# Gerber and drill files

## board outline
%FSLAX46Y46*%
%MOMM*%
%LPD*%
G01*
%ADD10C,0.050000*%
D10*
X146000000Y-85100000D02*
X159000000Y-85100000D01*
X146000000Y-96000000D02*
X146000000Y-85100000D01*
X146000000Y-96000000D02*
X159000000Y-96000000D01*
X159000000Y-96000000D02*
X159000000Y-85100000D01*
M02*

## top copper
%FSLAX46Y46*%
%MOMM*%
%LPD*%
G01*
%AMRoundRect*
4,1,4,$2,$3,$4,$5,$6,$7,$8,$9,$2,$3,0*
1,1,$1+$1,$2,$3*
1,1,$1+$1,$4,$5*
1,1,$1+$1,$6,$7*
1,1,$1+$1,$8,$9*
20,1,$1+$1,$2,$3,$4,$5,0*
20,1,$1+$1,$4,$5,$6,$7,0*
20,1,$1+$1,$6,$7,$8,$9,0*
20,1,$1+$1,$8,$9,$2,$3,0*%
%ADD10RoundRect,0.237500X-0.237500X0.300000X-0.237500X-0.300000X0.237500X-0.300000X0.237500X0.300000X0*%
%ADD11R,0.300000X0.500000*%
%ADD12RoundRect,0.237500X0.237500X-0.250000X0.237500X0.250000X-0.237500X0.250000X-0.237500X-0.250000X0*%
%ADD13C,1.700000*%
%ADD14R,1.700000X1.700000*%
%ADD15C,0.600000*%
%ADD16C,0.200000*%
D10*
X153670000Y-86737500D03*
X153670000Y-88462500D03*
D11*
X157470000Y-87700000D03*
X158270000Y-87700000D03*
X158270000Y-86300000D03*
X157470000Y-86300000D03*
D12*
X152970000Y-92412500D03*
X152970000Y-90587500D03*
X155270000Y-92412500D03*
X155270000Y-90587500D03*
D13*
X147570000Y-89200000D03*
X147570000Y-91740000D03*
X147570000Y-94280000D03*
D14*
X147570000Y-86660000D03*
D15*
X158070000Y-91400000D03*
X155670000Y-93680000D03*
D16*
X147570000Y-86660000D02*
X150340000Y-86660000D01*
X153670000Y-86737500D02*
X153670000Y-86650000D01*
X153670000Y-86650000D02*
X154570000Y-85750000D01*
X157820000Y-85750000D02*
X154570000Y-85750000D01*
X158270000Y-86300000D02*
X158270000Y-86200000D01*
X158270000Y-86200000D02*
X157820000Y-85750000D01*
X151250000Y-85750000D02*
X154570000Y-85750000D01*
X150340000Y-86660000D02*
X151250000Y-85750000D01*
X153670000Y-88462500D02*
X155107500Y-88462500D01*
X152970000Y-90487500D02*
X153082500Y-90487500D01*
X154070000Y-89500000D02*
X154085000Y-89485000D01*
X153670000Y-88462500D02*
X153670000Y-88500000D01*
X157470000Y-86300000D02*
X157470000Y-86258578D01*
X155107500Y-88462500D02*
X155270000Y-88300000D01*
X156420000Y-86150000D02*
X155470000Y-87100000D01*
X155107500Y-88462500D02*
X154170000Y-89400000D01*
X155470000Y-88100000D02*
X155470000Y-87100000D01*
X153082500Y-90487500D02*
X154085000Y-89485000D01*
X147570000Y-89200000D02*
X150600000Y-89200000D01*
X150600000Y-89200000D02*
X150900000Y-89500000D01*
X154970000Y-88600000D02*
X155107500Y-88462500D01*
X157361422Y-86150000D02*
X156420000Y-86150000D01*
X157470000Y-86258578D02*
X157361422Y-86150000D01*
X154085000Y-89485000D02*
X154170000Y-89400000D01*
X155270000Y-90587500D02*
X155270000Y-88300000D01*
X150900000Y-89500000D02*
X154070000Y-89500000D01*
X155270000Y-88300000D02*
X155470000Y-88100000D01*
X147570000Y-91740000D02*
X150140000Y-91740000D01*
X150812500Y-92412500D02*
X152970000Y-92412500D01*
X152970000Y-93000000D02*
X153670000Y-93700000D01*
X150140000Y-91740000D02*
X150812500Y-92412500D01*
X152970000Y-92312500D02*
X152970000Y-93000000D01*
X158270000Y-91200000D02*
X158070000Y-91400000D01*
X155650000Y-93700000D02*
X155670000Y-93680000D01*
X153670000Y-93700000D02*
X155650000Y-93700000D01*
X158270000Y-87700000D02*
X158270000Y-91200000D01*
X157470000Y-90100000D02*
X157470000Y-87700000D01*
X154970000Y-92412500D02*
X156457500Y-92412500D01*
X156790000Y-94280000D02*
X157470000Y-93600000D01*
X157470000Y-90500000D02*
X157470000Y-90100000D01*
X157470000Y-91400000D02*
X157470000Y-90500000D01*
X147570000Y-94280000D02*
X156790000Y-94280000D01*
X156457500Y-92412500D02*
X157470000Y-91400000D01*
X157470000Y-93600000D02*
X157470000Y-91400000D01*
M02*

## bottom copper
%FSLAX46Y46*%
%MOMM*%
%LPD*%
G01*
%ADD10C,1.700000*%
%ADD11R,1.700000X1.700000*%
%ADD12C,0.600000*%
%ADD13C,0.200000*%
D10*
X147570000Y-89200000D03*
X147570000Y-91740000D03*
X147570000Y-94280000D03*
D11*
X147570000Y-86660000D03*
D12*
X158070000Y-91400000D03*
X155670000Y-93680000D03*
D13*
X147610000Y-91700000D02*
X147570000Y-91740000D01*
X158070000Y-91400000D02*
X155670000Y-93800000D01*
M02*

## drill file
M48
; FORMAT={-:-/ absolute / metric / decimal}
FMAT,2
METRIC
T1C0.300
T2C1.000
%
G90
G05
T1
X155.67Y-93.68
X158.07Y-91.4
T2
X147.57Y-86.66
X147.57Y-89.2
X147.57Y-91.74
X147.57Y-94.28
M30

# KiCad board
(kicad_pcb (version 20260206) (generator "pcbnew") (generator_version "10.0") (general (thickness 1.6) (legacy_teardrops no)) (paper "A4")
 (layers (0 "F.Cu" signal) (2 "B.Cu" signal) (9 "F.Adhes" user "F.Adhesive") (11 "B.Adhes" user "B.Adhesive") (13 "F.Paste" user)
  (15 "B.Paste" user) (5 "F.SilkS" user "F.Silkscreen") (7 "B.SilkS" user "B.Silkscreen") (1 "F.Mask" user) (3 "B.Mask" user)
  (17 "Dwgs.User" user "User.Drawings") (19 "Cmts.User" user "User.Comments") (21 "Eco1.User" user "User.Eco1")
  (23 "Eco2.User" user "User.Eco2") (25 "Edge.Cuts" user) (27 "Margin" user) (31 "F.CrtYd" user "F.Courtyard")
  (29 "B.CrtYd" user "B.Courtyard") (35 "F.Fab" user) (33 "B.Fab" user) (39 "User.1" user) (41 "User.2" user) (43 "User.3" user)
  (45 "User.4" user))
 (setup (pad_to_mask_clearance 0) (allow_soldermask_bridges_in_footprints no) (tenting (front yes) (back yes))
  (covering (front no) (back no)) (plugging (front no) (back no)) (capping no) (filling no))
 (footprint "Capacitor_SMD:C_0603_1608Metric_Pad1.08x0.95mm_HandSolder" (layer "F.Cu") (at 153.67 87.6 -90)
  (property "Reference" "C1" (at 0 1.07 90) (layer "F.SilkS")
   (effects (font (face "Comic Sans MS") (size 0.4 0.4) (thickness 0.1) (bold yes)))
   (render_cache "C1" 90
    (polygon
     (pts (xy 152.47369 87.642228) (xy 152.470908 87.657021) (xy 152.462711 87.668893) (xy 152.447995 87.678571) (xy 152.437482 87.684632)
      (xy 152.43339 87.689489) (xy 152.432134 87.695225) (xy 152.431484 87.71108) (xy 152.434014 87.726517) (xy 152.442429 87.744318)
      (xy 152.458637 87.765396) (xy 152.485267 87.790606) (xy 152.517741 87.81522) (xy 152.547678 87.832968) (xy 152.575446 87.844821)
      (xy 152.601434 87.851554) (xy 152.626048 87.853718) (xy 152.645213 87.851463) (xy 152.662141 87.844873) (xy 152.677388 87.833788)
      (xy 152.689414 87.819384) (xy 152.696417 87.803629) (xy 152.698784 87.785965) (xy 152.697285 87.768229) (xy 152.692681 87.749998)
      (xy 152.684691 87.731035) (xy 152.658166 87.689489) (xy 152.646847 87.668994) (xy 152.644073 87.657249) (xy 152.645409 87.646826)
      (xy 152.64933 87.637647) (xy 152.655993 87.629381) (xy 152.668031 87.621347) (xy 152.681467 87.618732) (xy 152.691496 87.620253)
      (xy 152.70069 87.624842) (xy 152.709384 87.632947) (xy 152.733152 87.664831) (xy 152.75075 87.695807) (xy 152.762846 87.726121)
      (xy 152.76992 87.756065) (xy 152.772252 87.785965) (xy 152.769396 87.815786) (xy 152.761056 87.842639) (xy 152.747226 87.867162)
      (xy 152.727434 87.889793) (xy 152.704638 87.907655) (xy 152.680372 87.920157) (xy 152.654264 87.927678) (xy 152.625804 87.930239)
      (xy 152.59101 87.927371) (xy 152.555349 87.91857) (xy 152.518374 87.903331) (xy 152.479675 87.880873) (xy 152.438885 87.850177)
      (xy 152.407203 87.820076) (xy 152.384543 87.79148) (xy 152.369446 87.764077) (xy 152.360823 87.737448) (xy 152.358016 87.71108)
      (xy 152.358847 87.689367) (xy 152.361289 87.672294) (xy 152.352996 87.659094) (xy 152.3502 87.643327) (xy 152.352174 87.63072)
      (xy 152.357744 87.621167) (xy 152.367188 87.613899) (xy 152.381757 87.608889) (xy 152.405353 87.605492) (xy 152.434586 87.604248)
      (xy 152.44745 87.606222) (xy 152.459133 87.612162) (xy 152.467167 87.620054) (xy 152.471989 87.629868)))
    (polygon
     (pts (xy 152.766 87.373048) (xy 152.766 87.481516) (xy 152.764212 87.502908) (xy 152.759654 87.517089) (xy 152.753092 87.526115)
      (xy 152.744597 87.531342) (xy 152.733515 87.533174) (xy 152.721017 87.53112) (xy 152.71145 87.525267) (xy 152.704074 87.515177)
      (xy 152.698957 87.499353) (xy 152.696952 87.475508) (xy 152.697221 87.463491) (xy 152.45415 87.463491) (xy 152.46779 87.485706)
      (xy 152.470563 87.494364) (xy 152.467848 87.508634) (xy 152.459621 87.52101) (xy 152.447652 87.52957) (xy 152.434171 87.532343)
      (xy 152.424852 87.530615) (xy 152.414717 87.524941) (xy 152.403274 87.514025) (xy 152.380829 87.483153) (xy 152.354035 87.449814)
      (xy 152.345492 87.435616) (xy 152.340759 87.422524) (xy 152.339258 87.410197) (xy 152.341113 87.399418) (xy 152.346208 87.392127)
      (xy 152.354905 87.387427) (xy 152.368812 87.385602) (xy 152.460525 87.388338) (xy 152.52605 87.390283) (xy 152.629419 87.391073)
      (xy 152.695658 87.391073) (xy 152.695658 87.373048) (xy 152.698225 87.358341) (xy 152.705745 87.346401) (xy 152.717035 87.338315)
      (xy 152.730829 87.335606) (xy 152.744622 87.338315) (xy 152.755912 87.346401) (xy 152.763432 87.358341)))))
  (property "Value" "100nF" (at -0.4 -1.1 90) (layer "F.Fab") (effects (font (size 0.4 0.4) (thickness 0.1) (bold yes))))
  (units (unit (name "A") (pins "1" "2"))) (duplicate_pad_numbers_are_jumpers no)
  (pad "1" smd roundrect (at -0.8625 0 270) (size 1.075 0.95) (layers "F.Cu" "F.Mask" "F.Paste") (roundrect_rratio 0.25)
   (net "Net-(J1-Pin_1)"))
  (pad "2" smd roundrect (at 0.8625 0 270) (size 1.075 0.95) (layers "F.Cu" "F.Mask" "F.Paste") (roundrect_rratio 0.25)
   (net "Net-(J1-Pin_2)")))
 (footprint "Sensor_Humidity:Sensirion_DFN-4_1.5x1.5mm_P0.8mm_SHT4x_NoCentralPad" (layer "F.Cu") (at 157.87 87 90)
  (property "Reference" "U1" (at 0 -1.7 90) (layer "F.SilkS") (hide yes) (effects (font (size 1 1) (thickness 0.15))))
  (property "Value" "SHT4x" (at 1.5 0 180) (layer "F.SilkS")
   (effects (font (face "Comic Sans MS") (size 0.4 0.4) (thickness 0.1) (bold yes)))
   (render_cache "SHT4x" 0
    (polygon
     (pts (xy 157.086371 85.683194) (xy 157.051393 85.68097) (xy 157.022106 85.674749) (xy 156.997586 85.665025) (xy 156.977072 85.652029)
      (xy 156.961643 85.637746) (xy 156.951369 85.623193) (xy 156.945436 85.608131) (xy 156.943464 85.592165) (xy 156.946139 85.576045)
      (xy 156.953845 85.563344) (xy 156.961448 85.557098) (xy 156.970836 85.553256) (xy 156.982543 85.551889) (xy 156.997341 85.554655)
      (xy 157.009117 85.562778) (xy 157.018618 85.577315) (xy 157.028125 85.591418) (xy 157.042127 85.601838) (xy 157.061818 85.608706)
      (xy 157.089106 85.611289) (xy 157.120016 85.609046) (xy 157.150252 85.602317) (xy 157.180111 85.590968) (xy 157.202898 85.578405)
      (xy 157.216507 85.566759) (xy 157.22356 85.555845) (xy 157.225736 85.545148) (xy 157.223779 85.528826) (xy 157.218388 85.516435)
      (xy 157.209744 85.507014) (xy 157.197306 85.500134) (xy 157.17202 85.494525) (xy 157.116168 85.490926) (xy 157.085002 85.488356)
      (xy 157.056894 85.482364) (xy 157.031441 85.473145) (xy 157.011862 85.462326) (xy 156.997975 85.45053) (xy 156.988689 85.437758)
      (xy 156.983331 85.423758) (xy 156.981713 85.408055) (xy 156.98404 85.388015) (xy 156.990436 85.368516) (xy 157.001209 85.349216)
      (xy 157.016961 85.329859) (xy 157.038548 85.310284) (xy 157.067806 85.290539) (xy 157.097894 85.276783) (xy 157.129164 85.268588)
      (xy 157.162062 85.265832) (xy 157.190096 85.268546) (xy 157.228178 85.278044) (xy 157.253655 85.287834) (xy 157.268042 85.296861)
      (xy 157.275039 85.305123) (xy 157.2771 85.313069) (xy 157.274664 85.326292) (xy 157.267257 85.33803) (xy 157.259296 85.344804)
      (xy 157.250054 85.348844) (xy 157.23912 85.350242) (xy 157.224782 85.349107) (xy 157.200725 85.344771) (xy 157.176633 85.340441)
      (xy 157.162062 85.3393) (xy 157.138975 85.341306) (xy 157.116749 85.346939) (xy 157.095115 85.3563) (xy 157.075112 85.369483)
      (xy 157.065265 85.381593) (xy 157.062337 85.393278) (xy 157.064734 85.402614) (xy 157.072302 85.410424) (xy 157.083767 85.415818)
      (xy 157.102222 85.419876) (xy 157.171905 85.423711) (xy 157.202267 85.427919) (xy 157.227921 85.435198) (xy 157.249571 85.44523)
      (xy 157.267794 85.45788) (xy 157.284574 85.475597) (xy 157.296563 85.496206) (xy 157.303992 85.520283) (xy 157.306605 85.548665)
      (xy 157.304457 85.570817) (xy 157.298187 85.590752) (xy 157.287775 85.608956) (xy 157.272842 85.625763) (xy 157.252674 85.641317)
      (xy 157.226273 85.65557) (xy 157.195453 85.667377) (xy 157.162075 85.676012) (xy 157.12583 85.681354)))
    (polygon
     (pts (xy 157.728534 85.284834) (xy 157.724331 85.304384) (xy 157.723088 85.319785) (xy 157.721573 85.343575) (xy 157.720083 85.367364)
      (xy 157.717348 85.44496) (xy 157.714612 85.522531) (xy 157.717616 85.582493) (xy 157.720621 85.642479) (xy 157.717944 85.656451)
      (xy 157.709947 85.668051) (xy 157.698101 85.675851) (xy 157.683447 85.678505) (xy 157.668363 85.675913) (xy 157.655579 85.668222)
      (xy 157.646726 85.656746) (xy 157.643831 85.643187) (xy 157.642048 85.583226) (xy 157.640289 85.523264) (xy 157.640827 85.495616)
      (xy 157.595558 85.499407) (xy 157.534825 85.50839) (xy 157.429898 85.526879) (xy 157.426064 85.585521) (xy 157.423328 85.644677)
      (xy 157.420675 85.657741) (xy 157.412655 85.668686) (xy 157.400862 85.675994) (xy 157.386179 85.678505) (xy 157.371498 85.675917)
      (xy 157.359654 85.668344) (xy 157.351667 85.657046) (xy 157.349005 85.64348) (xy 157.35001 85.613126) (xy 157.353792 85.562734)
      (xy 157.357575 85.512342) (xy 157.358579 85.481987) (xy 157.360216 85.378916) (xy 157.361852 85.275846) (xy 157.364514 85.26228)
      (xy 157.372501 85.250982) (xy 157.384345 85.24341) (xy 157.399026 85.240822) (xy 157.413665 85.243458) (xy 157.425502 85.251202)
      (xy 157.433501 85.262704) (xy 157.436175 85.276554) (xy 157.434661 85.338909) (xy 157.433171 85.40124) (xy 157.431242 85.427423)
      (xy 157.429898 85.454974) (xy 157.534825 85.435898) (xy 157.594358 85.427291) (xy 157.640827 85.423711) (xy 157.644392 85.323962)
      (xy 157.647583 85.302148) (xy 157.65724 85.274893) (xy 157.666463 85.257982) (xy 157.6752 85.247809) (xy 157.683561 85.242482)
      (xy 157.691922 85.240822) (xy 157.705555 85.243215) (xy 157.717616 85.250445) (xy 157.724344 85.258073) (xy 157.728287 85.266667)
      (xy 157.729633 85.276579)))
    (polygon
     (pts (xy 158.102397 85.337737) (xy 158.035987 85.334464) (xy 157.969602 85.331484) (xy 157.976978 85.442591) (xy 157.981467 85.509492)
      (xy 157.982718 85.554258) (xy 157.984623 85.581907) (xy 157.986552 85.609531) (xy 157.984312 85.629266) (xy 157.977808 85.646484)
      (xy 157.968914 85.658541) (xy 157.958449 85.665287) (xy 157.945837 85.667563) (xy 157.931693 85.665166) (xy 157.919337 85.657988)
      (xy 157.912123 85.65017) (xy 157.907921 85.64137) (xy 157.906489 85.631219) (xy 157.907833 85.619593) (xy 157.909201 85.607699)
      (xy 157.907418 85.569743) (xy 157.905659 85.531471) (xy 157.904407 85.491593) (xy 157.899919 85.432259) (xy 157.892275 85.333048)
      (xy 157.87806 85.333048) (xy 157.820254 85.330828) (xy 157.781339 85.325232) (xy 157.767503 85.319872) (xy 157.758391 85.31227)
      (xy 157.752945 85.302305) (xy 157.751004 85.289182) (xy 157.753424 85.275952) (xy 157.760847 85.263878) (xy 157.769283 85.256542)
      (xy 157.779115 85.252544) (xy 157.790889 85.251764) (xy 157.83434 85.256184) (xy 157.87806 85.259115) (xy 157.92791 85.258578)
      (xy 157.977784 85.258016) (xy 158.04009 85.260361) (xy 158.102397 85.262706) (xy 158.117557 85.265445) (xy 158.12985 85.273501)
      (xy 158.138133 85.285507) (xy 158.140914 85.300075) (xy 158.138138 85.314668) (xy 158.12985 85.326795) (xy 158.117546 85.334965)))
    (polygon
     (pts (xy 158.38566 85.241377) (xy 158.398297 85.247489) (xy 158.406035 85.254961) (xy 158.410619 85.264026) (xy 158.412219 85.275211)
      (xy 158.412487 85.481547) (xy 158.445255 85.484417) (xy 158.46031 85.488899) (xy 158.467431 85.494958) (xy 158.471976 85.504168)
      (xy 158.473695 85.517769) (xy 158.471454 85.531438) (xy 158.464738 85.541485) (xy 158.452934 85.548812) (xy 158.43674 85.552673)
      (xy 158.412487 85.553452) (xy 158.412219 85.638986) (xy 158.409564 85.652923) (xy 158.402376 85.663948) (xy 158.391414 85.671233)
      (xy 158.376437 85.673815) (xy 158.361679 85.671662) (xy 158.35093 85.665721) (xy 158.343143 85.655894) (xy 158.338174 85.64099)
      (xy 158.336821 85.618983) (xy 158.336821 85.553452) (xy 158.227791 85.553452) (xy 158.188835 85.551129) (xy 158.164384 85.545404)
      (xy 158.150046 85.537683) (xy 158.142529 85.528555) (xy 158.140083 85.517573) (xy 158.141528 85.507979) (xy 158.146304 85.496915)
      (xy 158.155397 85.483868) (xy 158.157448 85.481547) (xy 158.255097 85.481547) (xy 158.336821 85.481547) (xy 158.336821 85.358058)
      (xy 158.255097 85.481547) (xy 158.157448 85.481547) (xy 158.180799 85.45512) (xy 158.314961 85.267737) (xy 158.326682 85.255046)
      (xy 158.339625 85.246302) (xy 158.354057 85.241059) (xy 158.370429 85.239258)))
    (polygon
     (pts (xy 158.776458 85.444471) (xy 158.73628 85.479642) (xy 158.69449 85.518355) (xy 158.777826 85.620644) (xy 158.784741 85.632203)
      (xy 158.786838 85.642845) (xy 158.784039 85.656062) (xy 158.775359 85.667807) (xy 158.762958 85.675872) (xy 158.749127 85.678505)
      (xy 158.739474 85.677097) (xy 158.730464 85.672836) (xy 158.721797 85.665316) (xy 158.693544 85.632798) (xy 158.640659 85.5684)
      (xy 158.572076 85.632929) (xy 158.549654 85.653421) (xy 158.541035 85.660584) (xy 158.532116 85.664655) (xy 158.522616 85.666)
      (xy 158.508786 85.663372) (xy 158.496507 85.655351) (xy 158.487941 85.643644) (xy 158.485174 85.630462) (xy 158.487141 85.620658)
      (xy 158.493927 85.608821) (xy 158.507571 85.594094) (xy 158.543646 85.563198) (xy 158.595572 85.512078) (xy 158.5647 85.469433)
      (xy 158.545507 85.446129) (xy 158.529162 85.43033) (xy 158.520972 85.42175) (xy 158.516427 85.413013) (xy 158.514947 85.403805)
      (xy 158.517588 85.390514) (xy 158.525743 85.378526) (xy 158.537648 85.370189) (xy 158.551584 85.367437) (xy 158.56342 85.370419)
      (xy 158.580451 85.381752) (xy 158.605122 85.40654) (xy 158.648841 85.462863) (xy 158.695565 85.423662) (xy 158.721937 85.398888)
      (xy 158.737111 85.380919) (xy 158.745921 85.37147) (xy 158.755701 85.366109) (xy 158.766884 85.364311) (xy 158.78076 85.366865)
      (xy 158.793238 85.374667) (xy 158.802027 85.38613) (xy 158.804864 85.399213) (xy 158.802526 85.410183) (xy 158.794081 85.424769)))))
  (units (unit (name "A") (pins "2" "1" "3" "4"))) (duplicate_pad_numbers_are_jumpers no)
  (pad "1" smd rect (at -0.7 -0.4 90) (size 0.5 0.3) (layers "F.Cu" "F.Mask" "F.Paste") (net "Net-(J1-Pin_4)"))
  (pad "2" smd rect (at -0.7 0.4 90) (size 0.5 0.3) (layers "F.Cu" "F.Mask" "F.Paste") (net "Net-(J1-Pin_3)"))
  (pad "3" smd rect (at 0.7 0.4 90) (size 0.5 0.3) (layers "F.Cu" "F.Mask" "F.Paste") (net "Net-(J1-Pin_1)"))
  (pad "4" smd rect (at 0.7 -0.4 90) (size 0.5 0.3) (layers "F.Cu" "F.Mask" "F.Paste") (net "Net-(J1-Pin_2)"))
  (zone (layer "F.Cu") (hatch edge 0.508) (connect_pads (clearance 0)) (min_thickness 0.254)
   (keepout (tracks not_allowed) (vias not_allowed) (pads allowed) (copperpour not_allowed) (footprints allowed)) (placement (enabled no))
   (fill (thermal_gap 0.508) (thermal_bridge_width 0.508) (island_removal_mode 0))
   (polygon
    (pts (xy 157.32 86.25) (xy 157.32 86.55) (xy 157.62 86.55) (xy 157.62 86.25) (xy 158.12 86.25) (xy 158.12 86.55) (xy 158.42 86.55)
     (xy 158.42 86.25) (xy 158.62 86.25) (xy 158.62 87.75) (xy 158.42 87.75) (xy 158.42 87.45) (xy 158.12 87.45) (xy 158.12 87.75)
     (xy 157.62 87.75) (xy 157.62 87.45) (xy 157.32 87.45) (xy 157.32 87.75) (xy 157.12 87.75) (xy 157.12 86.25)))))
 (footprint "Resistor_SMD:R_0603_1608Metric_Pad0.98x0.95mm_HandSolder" (layer "F.Cu") (at 152.97 91.5 90)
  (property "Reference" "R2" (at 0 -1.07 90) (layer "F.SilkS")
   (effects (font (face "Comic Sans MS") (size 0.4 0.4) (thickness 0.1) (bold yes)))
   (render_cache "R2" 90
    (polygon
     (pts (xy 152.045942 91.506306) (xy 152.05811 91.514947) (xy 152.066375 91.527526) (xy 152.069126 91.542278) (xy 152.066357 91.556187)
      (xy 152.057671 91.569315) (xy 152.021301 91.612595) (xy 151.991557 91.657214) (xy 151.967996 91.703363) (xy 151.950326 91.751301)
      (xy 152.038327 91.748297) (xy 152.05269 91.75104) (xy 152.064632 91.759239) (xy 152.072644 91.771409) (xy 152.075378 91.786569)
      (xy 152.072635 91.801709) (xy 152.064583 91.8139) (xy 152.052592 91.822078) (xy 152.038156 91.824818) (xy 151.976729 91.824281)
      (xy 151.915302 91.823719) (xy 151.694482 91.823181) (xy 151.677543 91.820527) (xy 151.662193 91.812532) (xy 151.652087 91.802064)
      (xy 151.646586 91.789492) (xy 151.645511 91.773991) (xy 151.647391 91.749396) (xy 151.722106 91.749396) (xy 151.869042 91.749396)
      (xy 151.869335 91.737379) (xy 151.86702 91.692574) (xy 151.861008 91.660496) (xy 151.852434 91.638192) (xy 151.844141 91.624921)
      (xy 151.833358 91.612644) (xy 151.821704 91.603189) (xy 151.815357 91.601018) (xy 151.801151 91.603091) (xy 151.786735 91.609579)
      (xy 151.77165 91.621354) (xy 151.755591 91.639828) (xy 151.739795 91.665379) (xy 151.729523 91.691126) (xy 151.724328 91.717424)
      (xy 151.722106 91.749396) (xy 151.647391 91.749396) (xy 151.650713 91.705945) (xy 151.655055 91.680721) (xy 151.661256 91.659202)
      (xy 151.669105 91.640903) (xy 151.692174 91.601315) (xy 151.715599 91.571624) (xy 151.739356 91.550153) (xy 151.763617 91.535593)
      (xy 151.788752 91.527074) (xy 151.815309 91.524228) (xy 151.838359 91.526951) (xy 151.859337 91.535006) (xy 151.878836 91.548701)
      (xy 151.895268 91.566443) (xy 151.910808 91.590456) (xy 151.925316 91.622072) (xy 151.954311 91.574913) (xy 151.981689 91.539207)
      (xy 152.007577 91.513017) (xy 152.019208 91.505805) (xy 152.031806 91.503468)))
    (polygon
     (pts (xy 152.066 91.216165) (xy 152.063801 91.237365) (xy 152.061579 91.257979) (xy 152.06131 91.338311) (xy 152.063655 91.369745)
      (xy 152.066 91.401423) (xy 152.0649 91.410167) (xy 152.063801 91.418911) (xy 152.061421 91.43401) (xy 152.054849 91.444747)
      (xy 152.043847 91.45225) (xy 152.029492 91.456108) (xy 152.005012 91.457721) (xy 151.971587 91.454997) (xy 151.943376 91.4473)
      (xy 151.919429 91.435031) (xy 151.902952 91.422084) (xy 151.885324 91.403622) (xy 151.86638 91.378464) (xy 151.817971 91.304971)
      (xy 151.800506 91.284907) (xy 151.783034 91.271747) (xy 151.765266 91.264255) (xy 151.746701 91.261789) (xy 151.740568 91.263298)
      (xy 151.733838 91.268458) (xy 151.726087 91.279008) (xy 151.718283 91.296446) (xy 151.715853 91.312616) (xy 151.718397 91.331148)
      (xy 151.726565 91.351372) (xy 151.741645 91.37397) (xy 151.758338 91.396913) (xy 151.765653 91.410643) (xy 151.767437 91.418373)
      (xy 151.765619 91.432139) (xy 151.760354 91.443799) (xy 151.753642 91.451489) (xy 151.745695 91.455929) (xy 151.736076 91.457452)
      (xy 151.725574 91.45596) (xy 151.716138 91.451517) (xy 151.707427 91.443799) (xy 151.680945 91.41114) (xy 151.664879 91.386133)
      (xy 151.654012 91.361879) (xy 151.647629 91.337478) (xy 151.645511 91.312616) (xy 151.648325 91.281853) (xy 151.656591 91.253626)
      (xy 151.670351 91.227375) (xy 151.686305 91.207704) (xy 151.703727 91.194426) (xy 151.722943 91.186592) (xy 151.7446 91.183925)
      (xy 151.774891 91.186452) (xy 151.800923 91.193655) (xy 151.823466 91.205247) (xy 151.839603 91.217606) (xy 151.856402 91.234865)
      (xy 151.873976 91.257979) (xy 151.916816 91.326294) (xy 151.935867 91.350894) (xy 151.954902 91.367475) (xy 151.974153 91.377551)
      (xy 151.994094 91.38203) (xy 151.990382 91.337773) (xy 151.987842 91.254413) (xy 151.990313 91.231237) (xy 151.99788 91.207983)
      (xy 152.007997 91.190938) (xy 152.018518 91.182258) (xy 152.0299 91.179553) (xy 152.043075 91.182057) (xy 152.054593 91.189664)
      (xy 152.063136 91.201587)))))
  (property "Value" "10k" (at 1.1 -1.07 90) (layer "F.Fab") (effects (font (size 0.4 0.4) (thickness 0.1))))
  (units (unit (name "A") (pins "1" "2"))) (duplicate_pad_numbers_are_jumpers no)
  (pad "1" smd roundrect (at -0.9125 0 90) (size 0.975 0.95) (layers "F.Cu" "F.Mask" "F.Paste") (roundrect_rratio 0.25)
   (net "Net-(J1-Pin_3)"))
  (pad "2" smd roundrect (at 0.9125 0 90) (size 0.975 0.95) (layers "F.Cu" "F.Mask" "F.Paste") (roundrect_rratio 0.25)
   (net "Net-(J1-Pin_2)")))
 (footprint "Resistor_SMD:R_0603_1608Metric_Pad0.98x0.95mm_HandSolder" (layer "F.Cu") (at 155.27 91.5 90)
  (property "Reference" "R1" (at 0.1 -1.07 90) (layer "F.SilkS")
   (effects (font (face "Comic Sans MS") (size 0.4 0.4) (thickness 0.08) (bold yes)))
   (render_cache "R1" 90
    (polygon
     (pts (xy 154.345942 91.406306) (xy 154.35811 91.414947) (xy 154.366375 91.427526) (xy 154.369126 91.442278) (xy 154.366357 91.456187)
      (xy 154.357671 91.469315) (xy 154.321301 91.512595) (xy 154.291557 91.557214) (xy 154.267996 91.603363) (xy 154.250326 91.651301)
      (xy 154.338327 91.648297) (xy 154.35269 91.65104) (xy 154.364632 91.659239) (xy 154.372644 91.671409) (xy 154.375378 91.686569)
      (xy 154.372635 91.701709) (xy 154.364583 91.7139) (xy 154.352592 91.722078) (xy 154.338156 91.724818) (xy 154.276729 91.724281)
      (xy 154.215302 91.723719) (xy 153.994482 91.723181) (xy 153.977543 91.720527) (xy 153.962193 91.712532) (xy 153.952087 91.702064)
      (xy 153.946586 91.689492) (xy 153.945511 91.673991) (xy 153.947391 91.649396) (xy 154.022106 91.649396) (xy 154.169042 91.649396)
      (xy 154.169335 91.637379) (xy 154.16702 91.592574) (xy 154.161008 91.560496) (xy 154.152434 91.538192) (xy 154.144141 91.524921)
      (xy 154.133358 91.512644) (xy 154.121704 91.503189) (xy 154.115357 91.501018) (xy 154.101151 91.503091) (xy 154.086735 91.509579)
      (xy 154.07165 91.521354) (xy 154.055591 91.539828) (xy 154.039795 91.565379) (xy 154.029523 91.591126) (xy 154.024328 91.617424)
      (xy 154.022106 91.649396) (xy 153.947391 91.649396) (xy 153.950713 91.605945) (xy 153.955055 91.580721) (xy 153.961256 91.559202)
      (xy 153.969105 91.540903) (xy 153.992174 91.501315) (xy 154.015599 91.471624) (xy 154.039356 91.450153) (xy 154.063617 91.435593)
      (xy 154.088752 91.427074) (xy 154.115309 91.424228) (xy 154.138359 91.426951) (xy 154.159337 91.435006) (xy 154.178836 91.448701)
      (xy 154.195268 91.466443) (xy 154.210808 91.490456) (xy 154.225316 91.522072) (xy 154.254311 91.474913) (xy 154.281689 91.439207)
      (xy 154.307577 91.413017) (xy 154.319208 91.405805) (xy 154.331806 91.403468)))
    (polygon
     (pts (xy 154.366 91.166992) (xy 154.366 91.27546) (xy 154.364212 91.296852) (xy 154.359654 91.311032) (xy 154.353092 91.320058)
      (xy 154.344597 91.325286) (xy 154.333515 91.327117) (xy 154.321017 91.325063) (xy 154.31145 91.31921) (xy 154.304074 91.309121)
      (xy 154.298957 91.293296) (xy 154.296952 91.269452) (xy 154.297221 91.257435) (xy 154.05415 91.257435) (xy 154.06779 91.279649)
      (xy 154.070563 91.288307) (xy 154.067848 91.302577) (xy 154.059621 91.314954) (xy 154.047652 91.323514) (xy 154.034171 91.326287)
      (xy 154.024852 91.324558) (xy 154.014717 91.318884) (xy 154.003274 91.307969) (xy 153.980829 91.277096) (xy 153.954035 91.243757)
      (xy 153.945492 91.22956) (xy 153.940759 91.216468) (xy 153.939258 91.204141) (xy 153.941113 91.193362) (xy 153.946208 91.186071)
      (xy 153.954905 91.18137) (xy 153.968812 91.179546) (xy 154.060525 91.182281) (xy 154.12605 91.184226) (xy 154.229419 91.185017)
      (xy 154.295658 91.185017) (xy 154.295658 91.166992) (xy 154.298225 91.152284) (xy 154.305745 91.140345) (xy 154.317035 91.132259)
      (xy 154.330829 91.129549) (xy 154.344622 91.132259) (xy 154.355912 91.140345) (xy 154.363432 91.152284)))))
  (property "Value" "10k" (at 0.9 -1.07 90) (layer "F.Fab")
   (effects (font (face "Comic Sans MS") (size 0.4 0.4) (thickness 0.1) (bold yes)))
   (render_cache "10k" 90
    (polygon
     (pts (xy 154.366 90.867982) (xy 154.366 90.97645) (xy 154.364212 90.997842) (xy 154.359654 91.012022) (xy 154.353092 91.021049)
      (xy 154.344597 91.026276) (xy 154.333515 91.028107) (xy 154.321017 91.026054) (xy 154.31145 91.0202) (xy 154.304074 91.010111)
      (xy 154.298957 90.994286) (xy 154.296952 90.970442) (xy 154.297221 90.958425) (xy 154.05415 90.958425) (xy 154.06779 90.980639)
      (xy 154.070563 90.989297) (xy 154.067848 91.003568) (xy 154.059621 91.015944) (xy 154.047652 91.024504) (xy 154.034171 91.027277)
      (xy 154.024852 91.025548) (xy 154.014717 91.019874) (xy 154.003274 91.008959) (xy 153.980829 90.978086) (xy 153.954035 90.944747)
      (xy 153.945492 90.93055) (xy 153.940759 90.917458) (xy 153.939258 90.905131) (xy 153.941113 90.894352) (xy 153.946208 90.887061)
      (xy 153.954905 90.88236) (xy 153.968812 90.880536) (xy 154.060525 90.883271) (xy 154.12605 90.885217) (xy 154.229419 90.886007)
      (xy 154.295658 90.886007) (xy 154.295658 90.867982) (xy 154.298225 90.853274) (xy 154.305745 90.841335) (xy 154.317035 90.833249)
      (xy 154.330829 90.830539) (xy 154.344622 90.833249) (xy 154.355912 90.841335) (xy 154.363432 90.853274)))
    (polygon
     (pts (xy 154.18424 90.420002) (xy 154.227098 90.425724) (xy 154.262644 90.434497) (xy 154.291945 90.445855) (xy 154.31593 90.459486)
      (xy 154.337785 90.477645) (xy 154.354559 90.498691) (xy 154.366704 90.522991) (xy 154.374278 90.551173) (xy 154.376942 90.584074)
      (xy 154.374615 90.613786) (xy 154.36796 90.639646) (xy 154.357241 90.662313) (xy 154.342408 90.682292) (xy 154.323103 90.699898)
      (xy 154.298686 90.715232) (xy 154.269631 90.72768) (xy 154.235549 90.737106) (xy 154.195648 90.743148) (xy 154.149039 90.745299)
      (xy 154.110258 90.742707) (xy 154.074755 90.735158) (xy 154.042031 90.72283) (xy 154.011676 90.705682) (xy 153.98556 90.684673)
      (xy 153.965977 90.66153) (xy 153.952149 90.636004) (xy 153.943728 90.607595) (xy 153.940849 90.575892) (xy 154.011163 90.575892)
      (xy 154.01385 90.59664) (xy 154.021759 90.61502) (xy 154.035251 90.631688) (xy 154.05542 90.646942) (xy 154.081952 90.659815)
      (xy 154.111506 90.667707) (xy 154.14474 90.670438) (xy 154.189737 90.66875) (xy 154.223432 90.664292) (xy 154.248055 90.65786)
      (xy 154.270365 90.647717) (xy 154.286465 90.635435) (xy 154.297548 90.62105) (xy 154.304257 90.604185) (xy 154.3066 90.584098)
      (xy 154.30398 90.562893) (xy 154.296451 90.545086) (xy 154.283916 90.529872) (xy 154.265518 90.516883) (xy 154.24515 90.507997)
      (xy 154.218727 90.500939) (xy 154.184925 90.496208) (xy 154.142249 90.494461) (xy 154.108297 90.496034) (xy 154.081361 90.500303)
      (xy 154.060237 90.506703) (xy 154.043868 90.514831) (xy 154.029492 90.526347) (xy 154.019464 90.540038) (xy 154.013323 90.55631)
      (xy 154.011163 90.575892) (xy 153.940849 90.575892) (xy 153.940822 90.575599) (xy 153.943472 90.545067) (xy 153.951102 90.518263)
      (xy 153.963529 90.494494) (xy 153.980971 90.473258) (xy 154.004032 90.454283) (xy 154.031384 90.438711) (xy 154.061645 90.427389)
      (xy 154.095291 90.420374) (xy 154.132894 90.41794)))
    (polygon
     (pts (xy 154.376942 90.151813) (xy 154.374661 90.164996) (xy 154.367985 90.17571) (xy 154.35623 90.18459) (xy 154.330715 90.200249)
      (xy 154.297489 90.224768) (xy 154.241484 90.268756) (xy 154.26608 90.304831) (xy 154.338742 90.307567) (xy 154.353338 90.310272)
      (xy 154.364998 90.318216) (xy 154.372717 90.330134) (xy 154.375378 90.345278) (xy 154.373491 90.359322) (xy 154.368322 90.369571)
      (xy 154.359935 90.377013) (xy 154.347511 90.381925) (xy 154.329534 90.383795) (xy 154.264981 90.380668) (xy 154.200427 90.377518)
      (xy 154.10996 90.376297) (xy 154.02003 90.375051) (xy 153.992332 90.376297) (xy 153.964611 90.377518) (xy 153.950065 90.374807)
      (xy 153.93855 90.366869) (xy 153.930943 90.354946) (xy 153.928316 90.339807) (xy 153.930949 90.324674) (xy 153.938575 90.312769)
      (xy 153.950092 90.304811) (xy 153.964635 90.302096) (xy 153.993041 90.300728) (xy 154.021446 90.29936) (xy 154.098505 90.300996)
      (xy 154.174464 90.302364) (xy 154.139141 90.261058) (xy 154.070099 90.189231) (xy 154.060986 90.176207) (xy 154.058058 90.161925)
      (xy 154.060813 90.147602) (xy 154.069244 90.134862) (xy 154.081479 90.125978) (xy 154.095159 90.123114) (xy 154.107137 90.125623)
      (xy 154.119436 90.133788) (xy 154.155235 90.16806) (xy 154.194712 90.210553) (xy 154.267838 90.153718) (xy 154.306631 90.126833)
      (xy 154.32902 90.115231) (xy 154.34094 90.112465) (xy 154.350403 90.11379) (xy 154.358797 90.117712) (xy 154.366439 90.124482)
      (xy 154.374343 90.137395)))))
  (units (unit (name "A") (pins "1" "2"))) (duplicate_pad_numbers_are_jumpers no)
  (pad "1" smd roundrect (at -0.9125 0 90) (size 0.975 0.95) (layers "F.Cu" "F.Mask" "F.Paste") (roundrect_rratio 0.25)
   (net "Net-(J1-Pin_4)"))
  (pad "2" smd roundrect (at 0.9125 0 90) (size 0.975 0.95) (layers "F.Cu" "F.Mask" "F.Paste") (roundrect_rratio 0.25)
   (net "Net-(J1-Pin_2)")))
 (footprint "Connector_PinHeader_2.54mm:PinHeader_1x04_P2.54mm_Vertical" (layer "B.Cu") (at 147.57 86.66 180)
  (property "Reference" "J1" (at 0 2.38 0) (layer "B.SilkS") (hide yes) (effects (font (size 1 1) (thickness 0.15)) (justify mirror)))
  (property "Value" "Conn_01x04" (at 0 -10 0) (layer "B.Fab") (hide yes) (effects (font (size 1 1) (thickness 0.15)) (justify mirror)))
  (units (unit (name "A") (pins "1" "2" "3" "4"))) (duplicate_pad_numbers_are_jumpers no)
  (pad "2" thru_hole circle (at 0 -2.54 180) (size 1.7 1.7) (drill 1) (layers "*.Cu" "*.Mask") (remove_unused_layers no) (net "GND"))
  (pad "3" thru_hole circle (at 0 -5.08 180) (size 1.7 1.7) (drill 1) (layers "*.Cu" "*.Mask") (remove_unused_layers no) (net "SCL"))
  (pad "4" thru_hole circle (at 0 -7.62 180) (size 1.7 1.7) (drill 1) (layers "*.Cu" "*.Mask") (remove_unused_layers no) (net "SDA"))
  (pad "16" thru_hole rect (at 0 0 180) (size 1.7 1.7) (drill 1) (layers "*.Cu" "*.Mask") (remove_unused_layers no) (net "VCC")))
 (gr_line (start 146 85.1) (end 159 85.1) (stroke (width 0.05) (type default)) (layer "Edge.Cuts"))
 (gr_line (start 146 96) (end 146 85.1) (stroke (width 0.05) (type default)) (layer "Edge.Cuts"))
 (gr_line (start 146 96) (end 159 96) (stroke (width 0.05) (type default)) (layer "Edge.Cuts"))
 (gr_line (start 159 96) (end 159 85.1) (stroke (width 0.05) (type default)) (layer "Edge.Cuts"))
 (segment (start 147.57 86.66) (end 150.34 86.66) (width 0.2) (layer "F.Cu") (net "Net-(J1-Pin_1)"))
 (segment (start 153.67 86.7375) (end 153.67 86.65) (width 0.2) (layer "F.Cu") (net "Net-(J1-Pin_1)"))
 (segment (start 153.67 86.65) (end 154.57 85.75) (width 0.2) (layer "F.Cu") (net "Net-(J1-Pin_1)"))
 (segment (start 157.82 85.75) (end 154.57 85.75) (width 0.2) (layer "F.Cu") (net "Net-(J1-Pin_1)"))
 (segment (start 158.27 86.3) (end 158.27 86.2) (width 0.2) (layer "F.Cu") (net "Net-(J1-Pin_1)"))
 (segment (start 158.27 86.2) (end 157.82 85.75) (width 0.2) (layer "F.Cu") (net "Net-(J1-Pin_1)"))
 (segment (start 151.25 85.75) (end 154.57 85.75) (width 0.2) (layer "F.Cu") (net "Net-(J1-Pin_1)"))
 (segment (start 150.34 86.66) (end 151.25 85.75) (width 0.2) (layer "F.Cu") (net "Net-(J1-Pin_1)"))
 (segment (start 153.67 88.4625) (end 155.1075 88.4625) (width 0.2) (layer "F.Cu") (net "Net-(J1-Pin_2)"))
 (segment (start 152.97 90.4875) (end 153.0825 90.4875) (width 0.2) (layer "F.Cu") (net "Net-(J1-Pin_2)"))
 (segment (start 154.07 89.5) (end 154.085 89.485) (width 0.2) (layer "F.Cu") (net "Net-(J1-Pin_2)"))
 (segment (start 153.67 88.4625) (end 153.67 88.5) (width 0.2) (layer "F.Cu") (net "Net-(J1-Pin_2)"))
 (segment (start 157.47 86.3) (end 157.47 86.258578) (width 0.2) (layer "F.Cu") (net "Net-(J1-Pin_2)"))
 (segment (start 155.1075 88.4625) (end 155.27 88.3) (width 0.2) (layer "F.Cu") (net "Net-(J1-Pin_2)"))
 (segment (start 156.42 86.15) (end 155.47 87.1) (width 0.2) (layer "F.Cu") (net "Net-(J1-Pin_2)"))
 (segment (start 155.1075 88.4625) (end 154.17 89.4) (width 0.2) (layer "F.Cu") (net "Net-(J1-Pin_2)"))
 (segment (start 155.47 88.1) (end 155.47 87.1) (width 0.2) (layer "F.Cu") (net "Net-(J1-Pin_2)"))
 (segment (start 153.0825 90.4875) (end 154.085 89.485) (width 0.2) (layer "F.Cu") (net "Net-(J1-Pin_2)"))
 (segment (start 147.57 89.2) (end 150.6 89.2) (width 0.2) (layer "F.Cu") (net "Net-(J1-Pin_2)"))
 (segment (start 150.6 89.2) (end 150.9 89.5) (width 0.2) (layer "F.Cu") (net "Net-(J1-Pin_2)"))
 (segment (start 154.97 88.6) (end 155.1075 88.4625) (width 0.2) (layer "F.Cu") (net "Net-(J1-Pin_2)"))
 (segment (start 157.361422 86.15) (end 156.42 86.15) (width 0.2) (layer "F.Cu") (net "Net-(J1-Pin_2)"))
 (segment (start 157.47 86.258578) (end 157.361422 86.15) (width 0.2) (layer "F.Cu") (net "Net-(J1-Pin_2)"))
 (segment (start 154.085 89.485) (end 154.17 89.4) (width 0.2) (layer "F.Cu") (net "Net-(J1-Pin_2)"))
 (segment (start 155.27 90.5875) (end 155.27 88.3) (width 0.2) (layer "F.Cu") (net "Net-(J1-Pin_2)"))
 (segment (start 150.9 89.5) (end 154.07 89.5) (width 0.2) (layer "F.Cu") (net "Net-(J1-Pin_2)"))
 (segment (start 155.27 88.3) (end 155.47 88.1) (width 0.2) (layer "F.Cu") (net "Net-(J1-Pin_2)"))
 (segment (start 147.57 91.74) (end 150.14 91.74) (width 0.2) (layer "F.Cu") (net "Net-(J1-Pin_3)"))
 (segment (start 150.8125 92.4125) (end 152.97 92.4125) (width 0.2) (layer "F.Cu") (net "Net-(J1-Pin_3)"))
 (segment (start 152.97 93) (end 153.67 93.7) (width 0.2) (layer "F.Cu") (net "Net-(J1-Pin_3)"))
 (segment (start 150.14 91.74) (end 150.8125 92.4125) (width 0.2) (layer "F.Cu") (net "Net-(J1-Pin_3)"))
 (segment (start 152.97 92.3125) (end 152.97 93) (width 0.2) (layer "F.Cu") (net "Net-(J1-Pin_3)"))
 (segment (start 158.27 91.2) (end 158.07 91.4) (width 0.2) (layer "F.Cu") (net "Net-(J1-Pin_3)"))
 (segment (start 155.65 93.7) (end 155.67 93.68) (width 0.2) (layer "F.Cu") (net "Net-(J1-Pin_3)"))
 (segment (start 153.67 93.7) (end 155.65 93.7) (width 0.2) (layer "F.Cu") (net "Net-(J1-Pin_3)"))
 (segment (start 158.27 87.7) (end 158.27 91.2) (width 0.2) (layer "F.Cu") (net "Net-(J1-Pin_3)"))
 (via (at 158.07 91.4) (size 0.6) (drill 0.3) (layers "F.Cu" "B.Cu") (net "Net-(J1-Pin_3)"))
 (via (at 155.67 93.68) (size 0.6) (drill 0.3) (layers "F.Cu" "B.Cu") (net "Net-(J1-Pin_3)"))
 (segment (start 147.61 91.7) (end 147.57 91.74) (width 0.2) (layer "B.Cu") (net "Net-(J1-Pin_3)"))
 (segment (start 158.07 91.4) (end 155.67 93.8) (width 0.2) (layer "B.Cu") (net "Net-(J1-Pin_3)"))
 (segment (start 157.47 90.1) (end 157.47 87.7) (width 0.2) (layer "F.Cu") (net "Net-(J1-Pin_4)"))
 (segment (start 154.97 92.4125) (end 156.4575 92.4125) (width 0.2) (layer "F.Cu") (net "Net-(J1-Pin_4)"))
 (segment (start 156.79 94.28) (end 157.47 93.6) (width 0.2) (layer "F.Cu") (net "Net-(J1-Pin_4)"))
 (segment (start 157.47 90.5) (end 157.47 90.1) (width 0.2) (layer "F.Cu") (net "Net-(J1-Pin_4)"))
 (segment (start 157.47 91.4) (end 157.47 90.5) (width 0.2) (layer "F.Cu") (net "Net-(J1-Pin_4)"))
 (segment (start 147.57 94.28) (end 156.79 94.28) (width 0.2) (layer "F.Cu") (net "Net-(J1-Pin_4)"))
 (segment (start 156.4575 92.4125) (end 157.47 91.4) (width 0.2) (layer "F.Cu") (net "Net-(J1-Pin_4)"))
 (segment (start 157.47 93.6) (end 157.47 91.4) (width 0.2) (layer "F.Cu") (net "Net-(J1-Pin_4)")))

